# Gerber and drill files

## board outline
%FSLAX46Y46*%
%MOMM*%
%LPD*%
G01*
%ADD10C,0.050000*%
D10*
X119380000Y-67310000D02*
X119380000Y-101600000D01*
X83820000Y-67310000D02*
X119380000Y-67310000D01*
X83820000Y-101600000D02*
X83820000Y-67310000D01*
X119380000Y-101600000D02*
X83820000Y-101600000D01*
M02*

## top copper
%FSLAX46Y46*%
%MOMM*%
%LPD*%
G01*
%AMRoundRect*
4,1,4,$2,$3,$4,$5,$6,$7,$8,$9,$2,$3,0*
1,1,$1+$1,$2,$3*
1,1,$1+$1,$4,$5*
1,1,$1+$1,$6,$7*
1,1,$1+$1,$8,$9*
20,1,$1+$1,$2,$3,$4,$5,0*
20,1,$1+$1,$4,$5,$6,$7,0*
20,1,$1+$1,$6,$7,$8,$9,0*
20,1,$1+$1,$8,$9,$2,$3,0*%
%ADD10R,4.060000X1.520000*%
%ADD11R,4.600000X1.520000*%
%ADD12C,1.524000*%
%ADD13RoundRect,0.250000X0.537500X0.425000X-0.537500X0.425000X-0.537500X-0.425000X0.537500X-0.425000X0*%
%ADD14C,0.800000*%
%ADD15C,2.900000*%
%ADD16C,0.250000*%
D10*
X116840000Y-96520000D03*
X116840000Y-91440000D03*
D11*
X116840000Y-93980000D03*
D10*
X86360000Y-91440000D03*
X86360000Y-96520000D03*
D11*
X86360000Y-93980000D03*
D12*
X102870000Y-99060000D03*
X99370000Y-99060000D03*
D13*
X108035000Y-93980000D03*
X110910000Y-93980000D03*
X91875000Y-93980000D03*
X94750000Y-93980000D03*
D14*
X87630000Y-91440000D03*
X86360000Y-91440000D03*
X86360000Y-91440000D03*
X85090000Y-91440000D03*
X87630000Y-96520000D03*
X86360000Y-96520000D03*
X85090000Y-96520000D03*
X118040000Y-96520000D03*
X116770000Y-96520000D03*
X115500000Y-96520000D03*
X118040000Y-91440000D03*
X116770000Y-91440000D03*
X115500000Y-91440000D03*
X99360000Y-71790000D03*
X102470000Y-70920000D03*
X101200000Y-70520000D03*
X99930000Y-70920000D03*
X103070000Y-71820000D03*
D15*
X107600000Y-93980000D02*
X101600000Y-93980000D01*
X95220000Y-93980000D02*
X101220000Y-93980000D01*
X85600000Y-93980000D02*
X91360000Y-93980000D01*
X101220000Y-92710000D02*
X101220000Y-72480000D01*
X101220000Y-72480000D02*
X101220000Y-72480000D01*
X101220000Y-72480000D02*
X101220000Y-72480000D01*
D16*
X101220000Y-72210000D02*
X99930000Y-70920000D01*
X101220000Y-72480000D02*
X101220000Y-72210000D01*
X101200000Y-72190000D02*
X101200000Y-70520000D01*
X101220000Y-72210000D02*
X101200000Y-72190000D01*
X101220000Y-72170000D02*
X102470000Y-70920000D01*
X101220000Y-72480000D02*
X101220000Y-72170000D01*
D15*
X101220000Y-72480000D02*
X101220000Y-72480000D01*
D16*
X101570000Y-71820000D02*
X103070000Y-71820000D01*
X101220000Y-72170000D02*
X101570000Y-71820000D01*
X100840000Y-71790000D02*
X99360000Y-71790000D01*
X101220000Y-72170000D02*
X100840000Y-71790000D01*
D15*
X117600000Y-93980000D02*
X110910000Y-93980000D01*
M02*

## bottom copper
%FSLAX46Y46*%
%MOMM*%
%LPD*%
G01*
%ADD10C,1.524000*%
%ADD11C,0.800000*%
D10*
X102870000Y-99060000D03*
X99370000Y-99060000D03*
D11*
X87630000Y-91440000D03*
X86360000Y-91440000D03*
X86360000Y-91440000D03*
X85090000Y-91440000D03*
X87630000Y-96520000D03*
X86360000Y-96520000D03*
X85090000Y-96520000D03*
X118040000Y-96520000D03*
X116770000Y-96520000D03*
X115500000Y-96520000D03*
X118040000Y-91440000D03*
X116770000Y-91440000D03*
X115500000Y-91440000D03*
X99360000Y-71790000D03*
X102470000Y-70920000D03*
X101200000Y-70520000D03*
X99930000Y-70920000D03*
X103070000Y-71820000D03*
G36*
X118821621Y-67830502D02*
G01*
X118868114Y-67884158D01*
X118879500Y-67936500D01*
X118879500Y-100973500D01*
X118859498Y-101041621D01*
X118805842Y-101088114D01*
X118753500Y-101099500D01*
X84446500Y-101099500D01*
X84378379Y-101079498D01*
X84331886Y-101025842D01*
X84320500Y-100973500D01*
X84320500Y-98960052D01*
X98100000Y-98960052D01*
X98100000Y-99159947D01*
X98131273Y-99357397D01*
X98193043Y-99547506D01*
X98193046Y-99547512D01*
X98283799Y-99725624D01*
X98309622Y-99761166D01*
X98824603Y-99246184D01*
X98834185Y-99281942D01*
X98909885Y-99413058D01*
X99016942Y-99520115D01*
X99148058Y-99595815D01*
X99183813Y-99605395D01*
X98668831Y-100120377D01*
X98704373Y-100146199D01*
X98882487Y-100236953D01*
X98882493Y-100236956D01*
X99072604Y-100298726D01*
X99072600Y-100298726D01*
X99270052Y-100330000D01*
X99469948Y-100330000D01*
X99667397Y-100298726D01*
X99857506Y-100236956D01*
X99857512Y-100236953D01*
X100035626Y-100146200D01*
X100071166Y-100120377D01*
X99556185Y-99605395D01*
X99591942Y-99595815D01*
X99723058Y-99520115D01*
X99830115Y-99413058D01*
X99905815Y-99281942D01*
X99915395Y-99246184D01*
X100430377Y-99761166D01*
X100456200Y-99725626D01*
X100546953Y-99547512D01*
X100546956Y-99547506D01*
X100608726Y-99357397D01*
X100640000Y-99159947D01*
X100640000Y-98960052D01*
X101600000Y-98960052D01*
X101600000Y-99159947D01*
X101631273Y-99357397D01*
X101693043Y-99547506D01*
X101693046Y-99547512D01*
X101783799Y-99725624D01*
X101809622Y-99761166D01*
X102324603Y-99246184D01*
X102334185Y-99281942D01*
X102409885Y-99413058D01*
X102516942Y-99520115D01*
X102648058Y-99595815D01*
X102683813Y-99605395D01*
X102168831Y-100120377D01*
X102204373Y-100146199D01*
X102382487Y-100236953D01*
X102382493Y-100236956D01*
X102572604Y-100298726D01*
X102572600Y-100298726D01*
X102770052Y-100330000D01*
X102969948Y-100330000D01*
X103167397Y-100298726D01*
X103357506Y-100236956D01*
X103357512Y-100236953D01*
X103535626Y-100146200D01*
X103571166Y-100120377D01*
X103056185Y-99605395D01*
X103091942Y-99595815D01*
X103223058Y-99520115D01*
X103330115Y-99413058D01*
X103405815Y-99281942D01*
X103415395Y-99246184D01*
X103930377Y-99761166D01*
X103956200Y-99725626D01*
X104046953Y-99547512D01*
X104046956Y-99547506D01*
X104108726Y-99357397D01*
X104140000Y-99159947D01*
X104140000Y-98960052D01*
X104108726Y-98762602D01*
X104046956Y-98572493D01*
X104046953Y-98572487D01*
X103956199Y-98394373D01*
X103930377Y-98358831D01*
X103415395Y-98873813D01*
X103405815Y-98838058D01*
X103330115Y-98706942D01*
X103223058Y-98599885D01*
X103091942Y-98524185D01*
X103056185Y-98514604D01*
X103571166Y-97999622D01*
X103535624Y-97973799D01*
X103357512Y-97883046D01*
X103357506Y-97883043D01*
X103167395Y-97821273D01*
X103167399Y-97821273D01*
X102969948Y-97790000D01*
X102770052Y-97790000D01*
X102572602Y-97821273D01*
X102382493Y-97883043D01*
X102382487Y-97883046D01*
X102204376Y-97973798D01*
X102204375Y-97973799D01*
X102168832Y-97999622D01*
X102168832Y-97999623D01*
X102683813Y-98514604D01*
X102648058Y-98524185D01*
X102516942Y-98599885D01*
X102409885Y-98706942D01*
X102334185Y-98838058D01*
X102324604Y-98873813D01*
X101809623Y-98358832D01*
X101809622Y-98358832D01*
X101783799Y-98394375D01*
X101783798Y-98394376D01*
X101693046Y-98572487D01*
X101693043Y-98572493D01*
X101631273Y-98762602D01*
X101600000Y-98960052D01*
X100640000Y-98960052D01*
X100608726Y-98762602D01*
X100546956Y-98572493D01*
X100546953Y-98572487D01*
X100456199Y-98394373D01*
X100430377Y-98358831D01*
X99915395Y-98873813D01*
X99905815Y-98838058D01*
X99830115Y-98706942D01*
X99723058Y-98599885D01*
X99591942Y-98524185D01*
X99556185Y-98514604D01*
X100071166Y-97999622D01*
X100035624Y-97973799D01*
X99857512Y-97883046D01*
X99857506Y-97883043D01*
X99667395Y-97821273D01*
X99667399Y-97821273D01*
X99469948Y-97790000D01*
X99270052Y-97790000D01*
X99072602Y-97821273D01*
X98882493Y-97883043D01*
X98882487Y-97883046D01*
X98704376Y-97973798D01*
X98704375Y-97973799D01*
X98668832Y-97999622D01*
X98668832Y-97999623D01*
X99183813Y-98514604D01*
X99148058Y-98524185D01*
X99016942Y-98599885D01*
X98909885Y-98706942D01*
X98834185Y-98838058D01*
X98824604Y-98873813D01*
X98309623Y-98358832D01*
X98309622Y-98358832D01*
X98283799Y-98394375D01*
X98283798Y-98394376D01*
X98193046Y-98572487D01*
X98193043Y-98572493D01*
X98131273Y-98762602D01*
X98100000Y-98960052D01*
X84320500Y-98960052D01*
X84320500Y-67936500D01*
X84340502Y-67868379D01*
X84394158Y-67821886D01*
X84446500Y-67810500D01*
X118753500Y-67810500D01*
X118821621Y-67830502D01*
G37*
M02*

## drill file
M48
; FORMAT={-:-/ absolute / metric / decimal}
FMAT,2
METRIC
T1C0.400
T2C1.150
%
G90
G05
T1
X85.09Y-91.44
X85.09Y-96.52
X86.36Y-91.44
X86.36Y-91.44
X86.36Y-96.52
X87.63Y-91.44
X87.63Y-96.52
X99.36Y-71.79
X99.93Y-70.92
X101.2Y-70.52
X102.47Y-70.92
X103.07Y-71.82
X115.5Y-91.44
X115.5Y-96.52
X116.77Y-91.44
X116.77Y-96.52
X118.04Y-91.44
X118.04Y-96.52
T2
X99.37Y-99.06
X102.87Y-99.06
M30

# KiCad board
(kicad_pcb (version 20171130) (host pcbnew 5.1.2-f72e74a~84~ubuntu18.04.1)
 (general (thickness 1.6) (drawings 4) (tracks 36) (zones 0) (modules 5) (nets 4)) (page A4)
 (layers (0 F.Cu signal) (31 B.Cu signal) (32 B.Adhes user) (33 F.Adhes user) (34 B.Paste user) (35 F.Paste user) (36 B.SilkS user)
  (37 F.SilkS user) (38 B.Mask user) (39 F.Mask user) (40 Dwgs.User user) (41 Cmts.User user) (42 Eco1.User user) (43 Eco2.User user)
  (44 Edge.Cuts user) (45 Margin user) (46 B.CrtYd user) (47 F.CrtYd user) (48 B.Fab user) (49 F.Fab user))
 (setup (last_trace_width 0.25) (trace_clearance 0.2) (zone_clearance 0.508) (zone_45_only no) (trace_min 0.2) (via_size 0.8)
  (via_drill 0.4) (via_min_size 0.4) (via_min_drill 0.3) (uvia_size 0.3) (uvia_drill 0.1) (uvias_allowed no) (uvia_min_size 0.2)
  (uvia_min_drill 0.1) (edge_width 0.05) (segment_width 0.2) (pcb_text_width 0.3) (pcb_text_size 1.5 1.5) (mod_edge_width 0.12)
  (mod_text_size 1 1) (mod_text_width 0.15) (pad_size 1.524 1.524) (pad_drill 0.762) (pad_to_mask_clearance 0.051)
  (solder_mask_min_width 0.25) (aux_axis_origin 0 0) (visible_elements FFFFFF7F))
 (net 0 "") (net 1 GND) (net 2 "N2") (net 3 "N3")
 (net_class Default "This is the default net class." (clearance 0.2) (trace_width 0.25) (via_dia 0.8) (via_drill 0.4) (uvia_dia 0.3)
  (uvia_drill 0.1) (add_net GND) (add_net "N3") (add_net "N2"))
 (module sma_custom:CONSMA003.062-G (layer F.Cu) (at 120.65 96.52)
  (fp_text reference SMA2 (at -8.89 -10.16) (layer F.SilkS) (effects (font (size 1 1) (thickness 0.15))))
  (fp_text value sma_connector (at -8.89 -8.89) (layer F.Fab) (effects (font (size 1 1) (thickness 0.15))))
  (pad 3 smd rect (at -3.81 0) (size 4.06 1.52) (layers F.Cu F.Paste F.Mask) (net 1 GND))
  (pad 2 smd rect (at -3.81 -5.08) (size 4.06 1.52) (layers F.Cu F.Paste F.Mask) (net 1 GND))
  (pad 1 smd rect (at -3.81 -2.54) (size 4.6 1.52) (layers F.Cu F.Paste F.Mask) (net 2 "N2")))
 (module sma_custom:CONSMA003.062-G (layer F.Cu) (at 82.55 91.44 180)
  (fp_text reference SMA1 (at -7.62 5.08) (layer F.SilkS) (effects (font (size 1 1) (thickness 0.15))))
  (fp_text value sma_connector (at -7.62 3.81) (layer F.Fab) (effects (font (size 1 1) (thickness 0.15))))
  (pad 3 smd rect (at -3.81 0 180) (size 4.06 1.52) (layers F.Cu F.Paste F.Mask) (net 1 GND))
  (pad 2 smd rect (at -3.81 -5.08 180) (size 4.06 1.52) (layers F.Cu F.Paste F.Mask) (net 1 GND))
  (pad 1 smd rect (at -3.81 -2.54 180) (size 4.6 1.52) (layers F.Cu F.Paste F.Mask) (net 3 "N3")))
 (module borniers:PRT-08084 (layer F.Cu) (at 102.87 104.14)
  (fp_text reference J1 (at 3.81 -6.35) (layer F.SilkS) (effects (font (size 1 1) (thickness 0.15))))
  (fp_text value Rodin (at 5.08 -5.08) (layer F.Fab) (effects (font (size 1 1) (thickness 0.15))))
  (pad 2 thru_hole circle (at 0 -5.08) (size 1.524 1.524) (drill 1.15) (layers *.Cu *.Mask) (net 1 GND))
  (pad 1 thru_hole circle (at -3.5 -5.08) (size 1.524 1.524) (drill 1.15) (layers *.Cu *.Mask) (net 1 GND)))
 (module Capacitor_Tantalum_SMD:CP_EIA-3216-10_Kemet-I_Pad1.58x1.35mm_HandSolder (layer F.Cu) (at 109.4725 93.98 180)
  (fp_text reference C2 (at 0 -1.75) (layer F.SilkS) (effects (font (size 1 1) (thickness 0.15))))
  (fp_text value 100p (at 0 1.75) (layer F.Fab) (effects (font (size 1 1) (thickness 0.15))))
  (pad 2 smd roundrect (at 1.4375 0 180) (size 1.575 1.35) (layers F.Cu F.Paste F.Mask) (roundrect_rratio 0.185185) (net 1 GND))
  (pad 1 smd roundrect (at -1.4375 0 180) (size 1.575 1.35) (layers F.Cu F.Paste F.Mask) (roundrect_rratio 0.185185) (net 2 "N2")))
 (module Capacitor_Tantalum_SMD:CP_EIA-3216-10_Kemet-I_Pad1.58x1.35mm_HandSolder (layer F.Cu) (at 93.3125 93.98 180)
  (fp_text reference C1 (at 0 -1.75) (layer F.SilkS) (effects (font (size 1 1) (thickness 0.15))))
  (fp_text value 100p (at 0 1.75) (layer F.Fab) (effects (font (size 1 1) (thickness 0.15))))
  (pad 2 smd roundrect (at 1.4375 0 180) (size 1.575 1.35) (layers F.Cu F.Paste F.Mask) (roundrect_rratio 0.185185) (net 3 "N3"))
  (pad 1 smd roundrect (at -1.4375 0 180) (size 1.575 1.35) (layers F.Cu F.Paste F.Mask) (roundrect_rratio 0.185185) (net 1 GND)))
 (gr_line (start 119.38 67.31) (end 119.38 101.6) (layer Edge.Cuts) (width 0.05))
 (gr_line (start 83.82 67.31) (end 119.38 67.31) (layer Edge.Cuts) (width 0.05))
 (gr_line (start 83.82 101.6) (end 83.82 67.31) (layer Edge.Cuts) (width 0.05))
 (gr_line (start 119.38 101.6) (end 83.82 101.6) (layer Edge.Cuts) (width 0.05))
 (via (at 87.63 91.44) (size 0.8) (drill 0.4) (layers F.Cu B.Cu) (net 1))
 (via (at 86.36 91.44) (size 0.8) (drill 0.4) (layers F.Cu B.Cu) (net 1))
 (via (at 86.36 91.44) (size 0.8) (drill 0.4) (layers F.Cu B.Cu) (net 1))
 (via (at 85.09 91.44) (size 0.8) (drill 0.4) (layers F.Cu B.Cu) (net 1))
 (via (at 87.63 96.52) (size 0.8) (drill 0.4) (layers F.Cu B.Cu) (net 1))
 (via (at 86.36 96.52) (size 0.8) (drill 0.4) (layers F.Cu B.Cu) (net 1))
 (via (at 85.09 96.52) (size 0.8) (drill 0.4) (layers F.Cu B.Cu) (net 1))
 (via (at 118.04 96.52) (size 0.8) (drill 0.4) (layers F.Cu B.Cu) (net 1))
 (via (at 116.77 96.52) (size 0.8) (drill 0.4) (layers F.Cu B.Cu) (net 1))
 (via (at 115.5 96.52) (size 0.8) (drill 0.4) (layers F.Cu B.Cu) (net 1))
 (via (at 118.04 91.44) (size 0.8) (drill 0.4) (layers F.Cu B.Cu) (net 1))
 (via (at 116.77 91.44) (size 0.8) (drill 0.4) (layers F.Cu B.Cu) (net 1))
 (via (at 115.5 91.44) (size 0.8) (drill 0.4) (layers F.Cu B.Cu) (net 1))
 (via (at 99.36 71.79) (size 0.8) (drill 0.4) (layers F.Cu B.Cu) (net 1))
 (via (at 102.47 70.92) (size 0.8) (drill 0.4) (layers F.Cu B.Cu) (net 1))
 (via (at 101.2 70.52) (size 0.8) (drill 0.4) (layers F.Cu B.Cu) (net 1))
 (via (at 99.93 70.92) (size 0.8) (drill 0.4) (layers F.Cu B.Cu) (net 1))
 (segment (start 107.6 93.98) (end 101.6 93.98) (width 2.9) (layer F.Cu) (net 1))
 (segment (start 95.22 93.98) (end 101.22 93.98) (width 2.9) (layer F.Cu) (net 1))
 (segment (start 85.6 93.98) (end 91.36 93.98) (width 2.9) (layer F.Cu) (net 3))
 (segment (start 101.22 92.71) (end 101.22 72.48) (width 2.9) (layer F.Cu) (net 1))
 (segment (start 101.22 72.48) (end 101.22 72.48) (width 2.9) (layer F.Cu) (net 1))
 (segment (start 101.22 72.48) (end 101.22 72.48) (width 2.9) (layer F.Cu) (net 1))
 (segment (start 101.22 72.21) (end 99.93 70.92) (width 0.25) (layer F.Cu) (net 1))
 (segment (start 101.22 72.48) (end 101.22 72.21) (width 0.25) (layer F.Cu) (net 1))
 (segment (start 101.2 72.19) (end 101.2 70.52) (width 0.25) (layer F.Cu) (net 1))
 (segment (start 101.22 72.21) (end 101.2 72.19) (width 0.25) (layer F.Cu) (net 1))
 (segment (start 101.22 72.17) (end 102.47 70.92) (width 0.25) (layer F.Cu) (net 1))
 (segment (start 101.22 72.48) (end 101.22 72.17) (width 0.25) (layer F.Cu) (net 1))
 (segment (start 101.22 72.48) (end 101.22 72.48) (width 2.9) (layer F.Cu) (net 1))
 (via (at 103.07 71.82) (size 0.8) (drill 0.4) (layers F.Cu B.Cu) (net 1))
 (segment (start 101.57 71.82) (end 103.07 71.82) (width 0.25) (layer F.Cu) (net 1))
 (segment (start 101.22 72.17) (end 101.57 71.82) (width 0.25) (layer F.Cu) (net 1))
 (segment (start 100.84 71.79) (end 99.36 71.79) (width 0.25) (layer F.Cu) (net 1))
 (segment (start 101.22 72.17) (end 100.84 71.79) (width 0.25) (layer F.Cu) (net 1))
 (segment (start 117.6 93.98) (end 110.91 93.98) (width 2.9) (layer F.Cu) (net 2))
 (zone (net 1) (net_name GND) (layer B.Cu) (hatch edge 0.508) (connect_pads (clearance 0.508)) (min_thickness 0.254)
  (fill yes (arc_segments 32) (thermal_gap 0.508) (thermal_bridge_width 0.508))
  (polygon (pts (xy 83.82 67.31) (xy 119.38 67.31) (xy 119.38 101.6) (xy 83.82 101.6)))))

